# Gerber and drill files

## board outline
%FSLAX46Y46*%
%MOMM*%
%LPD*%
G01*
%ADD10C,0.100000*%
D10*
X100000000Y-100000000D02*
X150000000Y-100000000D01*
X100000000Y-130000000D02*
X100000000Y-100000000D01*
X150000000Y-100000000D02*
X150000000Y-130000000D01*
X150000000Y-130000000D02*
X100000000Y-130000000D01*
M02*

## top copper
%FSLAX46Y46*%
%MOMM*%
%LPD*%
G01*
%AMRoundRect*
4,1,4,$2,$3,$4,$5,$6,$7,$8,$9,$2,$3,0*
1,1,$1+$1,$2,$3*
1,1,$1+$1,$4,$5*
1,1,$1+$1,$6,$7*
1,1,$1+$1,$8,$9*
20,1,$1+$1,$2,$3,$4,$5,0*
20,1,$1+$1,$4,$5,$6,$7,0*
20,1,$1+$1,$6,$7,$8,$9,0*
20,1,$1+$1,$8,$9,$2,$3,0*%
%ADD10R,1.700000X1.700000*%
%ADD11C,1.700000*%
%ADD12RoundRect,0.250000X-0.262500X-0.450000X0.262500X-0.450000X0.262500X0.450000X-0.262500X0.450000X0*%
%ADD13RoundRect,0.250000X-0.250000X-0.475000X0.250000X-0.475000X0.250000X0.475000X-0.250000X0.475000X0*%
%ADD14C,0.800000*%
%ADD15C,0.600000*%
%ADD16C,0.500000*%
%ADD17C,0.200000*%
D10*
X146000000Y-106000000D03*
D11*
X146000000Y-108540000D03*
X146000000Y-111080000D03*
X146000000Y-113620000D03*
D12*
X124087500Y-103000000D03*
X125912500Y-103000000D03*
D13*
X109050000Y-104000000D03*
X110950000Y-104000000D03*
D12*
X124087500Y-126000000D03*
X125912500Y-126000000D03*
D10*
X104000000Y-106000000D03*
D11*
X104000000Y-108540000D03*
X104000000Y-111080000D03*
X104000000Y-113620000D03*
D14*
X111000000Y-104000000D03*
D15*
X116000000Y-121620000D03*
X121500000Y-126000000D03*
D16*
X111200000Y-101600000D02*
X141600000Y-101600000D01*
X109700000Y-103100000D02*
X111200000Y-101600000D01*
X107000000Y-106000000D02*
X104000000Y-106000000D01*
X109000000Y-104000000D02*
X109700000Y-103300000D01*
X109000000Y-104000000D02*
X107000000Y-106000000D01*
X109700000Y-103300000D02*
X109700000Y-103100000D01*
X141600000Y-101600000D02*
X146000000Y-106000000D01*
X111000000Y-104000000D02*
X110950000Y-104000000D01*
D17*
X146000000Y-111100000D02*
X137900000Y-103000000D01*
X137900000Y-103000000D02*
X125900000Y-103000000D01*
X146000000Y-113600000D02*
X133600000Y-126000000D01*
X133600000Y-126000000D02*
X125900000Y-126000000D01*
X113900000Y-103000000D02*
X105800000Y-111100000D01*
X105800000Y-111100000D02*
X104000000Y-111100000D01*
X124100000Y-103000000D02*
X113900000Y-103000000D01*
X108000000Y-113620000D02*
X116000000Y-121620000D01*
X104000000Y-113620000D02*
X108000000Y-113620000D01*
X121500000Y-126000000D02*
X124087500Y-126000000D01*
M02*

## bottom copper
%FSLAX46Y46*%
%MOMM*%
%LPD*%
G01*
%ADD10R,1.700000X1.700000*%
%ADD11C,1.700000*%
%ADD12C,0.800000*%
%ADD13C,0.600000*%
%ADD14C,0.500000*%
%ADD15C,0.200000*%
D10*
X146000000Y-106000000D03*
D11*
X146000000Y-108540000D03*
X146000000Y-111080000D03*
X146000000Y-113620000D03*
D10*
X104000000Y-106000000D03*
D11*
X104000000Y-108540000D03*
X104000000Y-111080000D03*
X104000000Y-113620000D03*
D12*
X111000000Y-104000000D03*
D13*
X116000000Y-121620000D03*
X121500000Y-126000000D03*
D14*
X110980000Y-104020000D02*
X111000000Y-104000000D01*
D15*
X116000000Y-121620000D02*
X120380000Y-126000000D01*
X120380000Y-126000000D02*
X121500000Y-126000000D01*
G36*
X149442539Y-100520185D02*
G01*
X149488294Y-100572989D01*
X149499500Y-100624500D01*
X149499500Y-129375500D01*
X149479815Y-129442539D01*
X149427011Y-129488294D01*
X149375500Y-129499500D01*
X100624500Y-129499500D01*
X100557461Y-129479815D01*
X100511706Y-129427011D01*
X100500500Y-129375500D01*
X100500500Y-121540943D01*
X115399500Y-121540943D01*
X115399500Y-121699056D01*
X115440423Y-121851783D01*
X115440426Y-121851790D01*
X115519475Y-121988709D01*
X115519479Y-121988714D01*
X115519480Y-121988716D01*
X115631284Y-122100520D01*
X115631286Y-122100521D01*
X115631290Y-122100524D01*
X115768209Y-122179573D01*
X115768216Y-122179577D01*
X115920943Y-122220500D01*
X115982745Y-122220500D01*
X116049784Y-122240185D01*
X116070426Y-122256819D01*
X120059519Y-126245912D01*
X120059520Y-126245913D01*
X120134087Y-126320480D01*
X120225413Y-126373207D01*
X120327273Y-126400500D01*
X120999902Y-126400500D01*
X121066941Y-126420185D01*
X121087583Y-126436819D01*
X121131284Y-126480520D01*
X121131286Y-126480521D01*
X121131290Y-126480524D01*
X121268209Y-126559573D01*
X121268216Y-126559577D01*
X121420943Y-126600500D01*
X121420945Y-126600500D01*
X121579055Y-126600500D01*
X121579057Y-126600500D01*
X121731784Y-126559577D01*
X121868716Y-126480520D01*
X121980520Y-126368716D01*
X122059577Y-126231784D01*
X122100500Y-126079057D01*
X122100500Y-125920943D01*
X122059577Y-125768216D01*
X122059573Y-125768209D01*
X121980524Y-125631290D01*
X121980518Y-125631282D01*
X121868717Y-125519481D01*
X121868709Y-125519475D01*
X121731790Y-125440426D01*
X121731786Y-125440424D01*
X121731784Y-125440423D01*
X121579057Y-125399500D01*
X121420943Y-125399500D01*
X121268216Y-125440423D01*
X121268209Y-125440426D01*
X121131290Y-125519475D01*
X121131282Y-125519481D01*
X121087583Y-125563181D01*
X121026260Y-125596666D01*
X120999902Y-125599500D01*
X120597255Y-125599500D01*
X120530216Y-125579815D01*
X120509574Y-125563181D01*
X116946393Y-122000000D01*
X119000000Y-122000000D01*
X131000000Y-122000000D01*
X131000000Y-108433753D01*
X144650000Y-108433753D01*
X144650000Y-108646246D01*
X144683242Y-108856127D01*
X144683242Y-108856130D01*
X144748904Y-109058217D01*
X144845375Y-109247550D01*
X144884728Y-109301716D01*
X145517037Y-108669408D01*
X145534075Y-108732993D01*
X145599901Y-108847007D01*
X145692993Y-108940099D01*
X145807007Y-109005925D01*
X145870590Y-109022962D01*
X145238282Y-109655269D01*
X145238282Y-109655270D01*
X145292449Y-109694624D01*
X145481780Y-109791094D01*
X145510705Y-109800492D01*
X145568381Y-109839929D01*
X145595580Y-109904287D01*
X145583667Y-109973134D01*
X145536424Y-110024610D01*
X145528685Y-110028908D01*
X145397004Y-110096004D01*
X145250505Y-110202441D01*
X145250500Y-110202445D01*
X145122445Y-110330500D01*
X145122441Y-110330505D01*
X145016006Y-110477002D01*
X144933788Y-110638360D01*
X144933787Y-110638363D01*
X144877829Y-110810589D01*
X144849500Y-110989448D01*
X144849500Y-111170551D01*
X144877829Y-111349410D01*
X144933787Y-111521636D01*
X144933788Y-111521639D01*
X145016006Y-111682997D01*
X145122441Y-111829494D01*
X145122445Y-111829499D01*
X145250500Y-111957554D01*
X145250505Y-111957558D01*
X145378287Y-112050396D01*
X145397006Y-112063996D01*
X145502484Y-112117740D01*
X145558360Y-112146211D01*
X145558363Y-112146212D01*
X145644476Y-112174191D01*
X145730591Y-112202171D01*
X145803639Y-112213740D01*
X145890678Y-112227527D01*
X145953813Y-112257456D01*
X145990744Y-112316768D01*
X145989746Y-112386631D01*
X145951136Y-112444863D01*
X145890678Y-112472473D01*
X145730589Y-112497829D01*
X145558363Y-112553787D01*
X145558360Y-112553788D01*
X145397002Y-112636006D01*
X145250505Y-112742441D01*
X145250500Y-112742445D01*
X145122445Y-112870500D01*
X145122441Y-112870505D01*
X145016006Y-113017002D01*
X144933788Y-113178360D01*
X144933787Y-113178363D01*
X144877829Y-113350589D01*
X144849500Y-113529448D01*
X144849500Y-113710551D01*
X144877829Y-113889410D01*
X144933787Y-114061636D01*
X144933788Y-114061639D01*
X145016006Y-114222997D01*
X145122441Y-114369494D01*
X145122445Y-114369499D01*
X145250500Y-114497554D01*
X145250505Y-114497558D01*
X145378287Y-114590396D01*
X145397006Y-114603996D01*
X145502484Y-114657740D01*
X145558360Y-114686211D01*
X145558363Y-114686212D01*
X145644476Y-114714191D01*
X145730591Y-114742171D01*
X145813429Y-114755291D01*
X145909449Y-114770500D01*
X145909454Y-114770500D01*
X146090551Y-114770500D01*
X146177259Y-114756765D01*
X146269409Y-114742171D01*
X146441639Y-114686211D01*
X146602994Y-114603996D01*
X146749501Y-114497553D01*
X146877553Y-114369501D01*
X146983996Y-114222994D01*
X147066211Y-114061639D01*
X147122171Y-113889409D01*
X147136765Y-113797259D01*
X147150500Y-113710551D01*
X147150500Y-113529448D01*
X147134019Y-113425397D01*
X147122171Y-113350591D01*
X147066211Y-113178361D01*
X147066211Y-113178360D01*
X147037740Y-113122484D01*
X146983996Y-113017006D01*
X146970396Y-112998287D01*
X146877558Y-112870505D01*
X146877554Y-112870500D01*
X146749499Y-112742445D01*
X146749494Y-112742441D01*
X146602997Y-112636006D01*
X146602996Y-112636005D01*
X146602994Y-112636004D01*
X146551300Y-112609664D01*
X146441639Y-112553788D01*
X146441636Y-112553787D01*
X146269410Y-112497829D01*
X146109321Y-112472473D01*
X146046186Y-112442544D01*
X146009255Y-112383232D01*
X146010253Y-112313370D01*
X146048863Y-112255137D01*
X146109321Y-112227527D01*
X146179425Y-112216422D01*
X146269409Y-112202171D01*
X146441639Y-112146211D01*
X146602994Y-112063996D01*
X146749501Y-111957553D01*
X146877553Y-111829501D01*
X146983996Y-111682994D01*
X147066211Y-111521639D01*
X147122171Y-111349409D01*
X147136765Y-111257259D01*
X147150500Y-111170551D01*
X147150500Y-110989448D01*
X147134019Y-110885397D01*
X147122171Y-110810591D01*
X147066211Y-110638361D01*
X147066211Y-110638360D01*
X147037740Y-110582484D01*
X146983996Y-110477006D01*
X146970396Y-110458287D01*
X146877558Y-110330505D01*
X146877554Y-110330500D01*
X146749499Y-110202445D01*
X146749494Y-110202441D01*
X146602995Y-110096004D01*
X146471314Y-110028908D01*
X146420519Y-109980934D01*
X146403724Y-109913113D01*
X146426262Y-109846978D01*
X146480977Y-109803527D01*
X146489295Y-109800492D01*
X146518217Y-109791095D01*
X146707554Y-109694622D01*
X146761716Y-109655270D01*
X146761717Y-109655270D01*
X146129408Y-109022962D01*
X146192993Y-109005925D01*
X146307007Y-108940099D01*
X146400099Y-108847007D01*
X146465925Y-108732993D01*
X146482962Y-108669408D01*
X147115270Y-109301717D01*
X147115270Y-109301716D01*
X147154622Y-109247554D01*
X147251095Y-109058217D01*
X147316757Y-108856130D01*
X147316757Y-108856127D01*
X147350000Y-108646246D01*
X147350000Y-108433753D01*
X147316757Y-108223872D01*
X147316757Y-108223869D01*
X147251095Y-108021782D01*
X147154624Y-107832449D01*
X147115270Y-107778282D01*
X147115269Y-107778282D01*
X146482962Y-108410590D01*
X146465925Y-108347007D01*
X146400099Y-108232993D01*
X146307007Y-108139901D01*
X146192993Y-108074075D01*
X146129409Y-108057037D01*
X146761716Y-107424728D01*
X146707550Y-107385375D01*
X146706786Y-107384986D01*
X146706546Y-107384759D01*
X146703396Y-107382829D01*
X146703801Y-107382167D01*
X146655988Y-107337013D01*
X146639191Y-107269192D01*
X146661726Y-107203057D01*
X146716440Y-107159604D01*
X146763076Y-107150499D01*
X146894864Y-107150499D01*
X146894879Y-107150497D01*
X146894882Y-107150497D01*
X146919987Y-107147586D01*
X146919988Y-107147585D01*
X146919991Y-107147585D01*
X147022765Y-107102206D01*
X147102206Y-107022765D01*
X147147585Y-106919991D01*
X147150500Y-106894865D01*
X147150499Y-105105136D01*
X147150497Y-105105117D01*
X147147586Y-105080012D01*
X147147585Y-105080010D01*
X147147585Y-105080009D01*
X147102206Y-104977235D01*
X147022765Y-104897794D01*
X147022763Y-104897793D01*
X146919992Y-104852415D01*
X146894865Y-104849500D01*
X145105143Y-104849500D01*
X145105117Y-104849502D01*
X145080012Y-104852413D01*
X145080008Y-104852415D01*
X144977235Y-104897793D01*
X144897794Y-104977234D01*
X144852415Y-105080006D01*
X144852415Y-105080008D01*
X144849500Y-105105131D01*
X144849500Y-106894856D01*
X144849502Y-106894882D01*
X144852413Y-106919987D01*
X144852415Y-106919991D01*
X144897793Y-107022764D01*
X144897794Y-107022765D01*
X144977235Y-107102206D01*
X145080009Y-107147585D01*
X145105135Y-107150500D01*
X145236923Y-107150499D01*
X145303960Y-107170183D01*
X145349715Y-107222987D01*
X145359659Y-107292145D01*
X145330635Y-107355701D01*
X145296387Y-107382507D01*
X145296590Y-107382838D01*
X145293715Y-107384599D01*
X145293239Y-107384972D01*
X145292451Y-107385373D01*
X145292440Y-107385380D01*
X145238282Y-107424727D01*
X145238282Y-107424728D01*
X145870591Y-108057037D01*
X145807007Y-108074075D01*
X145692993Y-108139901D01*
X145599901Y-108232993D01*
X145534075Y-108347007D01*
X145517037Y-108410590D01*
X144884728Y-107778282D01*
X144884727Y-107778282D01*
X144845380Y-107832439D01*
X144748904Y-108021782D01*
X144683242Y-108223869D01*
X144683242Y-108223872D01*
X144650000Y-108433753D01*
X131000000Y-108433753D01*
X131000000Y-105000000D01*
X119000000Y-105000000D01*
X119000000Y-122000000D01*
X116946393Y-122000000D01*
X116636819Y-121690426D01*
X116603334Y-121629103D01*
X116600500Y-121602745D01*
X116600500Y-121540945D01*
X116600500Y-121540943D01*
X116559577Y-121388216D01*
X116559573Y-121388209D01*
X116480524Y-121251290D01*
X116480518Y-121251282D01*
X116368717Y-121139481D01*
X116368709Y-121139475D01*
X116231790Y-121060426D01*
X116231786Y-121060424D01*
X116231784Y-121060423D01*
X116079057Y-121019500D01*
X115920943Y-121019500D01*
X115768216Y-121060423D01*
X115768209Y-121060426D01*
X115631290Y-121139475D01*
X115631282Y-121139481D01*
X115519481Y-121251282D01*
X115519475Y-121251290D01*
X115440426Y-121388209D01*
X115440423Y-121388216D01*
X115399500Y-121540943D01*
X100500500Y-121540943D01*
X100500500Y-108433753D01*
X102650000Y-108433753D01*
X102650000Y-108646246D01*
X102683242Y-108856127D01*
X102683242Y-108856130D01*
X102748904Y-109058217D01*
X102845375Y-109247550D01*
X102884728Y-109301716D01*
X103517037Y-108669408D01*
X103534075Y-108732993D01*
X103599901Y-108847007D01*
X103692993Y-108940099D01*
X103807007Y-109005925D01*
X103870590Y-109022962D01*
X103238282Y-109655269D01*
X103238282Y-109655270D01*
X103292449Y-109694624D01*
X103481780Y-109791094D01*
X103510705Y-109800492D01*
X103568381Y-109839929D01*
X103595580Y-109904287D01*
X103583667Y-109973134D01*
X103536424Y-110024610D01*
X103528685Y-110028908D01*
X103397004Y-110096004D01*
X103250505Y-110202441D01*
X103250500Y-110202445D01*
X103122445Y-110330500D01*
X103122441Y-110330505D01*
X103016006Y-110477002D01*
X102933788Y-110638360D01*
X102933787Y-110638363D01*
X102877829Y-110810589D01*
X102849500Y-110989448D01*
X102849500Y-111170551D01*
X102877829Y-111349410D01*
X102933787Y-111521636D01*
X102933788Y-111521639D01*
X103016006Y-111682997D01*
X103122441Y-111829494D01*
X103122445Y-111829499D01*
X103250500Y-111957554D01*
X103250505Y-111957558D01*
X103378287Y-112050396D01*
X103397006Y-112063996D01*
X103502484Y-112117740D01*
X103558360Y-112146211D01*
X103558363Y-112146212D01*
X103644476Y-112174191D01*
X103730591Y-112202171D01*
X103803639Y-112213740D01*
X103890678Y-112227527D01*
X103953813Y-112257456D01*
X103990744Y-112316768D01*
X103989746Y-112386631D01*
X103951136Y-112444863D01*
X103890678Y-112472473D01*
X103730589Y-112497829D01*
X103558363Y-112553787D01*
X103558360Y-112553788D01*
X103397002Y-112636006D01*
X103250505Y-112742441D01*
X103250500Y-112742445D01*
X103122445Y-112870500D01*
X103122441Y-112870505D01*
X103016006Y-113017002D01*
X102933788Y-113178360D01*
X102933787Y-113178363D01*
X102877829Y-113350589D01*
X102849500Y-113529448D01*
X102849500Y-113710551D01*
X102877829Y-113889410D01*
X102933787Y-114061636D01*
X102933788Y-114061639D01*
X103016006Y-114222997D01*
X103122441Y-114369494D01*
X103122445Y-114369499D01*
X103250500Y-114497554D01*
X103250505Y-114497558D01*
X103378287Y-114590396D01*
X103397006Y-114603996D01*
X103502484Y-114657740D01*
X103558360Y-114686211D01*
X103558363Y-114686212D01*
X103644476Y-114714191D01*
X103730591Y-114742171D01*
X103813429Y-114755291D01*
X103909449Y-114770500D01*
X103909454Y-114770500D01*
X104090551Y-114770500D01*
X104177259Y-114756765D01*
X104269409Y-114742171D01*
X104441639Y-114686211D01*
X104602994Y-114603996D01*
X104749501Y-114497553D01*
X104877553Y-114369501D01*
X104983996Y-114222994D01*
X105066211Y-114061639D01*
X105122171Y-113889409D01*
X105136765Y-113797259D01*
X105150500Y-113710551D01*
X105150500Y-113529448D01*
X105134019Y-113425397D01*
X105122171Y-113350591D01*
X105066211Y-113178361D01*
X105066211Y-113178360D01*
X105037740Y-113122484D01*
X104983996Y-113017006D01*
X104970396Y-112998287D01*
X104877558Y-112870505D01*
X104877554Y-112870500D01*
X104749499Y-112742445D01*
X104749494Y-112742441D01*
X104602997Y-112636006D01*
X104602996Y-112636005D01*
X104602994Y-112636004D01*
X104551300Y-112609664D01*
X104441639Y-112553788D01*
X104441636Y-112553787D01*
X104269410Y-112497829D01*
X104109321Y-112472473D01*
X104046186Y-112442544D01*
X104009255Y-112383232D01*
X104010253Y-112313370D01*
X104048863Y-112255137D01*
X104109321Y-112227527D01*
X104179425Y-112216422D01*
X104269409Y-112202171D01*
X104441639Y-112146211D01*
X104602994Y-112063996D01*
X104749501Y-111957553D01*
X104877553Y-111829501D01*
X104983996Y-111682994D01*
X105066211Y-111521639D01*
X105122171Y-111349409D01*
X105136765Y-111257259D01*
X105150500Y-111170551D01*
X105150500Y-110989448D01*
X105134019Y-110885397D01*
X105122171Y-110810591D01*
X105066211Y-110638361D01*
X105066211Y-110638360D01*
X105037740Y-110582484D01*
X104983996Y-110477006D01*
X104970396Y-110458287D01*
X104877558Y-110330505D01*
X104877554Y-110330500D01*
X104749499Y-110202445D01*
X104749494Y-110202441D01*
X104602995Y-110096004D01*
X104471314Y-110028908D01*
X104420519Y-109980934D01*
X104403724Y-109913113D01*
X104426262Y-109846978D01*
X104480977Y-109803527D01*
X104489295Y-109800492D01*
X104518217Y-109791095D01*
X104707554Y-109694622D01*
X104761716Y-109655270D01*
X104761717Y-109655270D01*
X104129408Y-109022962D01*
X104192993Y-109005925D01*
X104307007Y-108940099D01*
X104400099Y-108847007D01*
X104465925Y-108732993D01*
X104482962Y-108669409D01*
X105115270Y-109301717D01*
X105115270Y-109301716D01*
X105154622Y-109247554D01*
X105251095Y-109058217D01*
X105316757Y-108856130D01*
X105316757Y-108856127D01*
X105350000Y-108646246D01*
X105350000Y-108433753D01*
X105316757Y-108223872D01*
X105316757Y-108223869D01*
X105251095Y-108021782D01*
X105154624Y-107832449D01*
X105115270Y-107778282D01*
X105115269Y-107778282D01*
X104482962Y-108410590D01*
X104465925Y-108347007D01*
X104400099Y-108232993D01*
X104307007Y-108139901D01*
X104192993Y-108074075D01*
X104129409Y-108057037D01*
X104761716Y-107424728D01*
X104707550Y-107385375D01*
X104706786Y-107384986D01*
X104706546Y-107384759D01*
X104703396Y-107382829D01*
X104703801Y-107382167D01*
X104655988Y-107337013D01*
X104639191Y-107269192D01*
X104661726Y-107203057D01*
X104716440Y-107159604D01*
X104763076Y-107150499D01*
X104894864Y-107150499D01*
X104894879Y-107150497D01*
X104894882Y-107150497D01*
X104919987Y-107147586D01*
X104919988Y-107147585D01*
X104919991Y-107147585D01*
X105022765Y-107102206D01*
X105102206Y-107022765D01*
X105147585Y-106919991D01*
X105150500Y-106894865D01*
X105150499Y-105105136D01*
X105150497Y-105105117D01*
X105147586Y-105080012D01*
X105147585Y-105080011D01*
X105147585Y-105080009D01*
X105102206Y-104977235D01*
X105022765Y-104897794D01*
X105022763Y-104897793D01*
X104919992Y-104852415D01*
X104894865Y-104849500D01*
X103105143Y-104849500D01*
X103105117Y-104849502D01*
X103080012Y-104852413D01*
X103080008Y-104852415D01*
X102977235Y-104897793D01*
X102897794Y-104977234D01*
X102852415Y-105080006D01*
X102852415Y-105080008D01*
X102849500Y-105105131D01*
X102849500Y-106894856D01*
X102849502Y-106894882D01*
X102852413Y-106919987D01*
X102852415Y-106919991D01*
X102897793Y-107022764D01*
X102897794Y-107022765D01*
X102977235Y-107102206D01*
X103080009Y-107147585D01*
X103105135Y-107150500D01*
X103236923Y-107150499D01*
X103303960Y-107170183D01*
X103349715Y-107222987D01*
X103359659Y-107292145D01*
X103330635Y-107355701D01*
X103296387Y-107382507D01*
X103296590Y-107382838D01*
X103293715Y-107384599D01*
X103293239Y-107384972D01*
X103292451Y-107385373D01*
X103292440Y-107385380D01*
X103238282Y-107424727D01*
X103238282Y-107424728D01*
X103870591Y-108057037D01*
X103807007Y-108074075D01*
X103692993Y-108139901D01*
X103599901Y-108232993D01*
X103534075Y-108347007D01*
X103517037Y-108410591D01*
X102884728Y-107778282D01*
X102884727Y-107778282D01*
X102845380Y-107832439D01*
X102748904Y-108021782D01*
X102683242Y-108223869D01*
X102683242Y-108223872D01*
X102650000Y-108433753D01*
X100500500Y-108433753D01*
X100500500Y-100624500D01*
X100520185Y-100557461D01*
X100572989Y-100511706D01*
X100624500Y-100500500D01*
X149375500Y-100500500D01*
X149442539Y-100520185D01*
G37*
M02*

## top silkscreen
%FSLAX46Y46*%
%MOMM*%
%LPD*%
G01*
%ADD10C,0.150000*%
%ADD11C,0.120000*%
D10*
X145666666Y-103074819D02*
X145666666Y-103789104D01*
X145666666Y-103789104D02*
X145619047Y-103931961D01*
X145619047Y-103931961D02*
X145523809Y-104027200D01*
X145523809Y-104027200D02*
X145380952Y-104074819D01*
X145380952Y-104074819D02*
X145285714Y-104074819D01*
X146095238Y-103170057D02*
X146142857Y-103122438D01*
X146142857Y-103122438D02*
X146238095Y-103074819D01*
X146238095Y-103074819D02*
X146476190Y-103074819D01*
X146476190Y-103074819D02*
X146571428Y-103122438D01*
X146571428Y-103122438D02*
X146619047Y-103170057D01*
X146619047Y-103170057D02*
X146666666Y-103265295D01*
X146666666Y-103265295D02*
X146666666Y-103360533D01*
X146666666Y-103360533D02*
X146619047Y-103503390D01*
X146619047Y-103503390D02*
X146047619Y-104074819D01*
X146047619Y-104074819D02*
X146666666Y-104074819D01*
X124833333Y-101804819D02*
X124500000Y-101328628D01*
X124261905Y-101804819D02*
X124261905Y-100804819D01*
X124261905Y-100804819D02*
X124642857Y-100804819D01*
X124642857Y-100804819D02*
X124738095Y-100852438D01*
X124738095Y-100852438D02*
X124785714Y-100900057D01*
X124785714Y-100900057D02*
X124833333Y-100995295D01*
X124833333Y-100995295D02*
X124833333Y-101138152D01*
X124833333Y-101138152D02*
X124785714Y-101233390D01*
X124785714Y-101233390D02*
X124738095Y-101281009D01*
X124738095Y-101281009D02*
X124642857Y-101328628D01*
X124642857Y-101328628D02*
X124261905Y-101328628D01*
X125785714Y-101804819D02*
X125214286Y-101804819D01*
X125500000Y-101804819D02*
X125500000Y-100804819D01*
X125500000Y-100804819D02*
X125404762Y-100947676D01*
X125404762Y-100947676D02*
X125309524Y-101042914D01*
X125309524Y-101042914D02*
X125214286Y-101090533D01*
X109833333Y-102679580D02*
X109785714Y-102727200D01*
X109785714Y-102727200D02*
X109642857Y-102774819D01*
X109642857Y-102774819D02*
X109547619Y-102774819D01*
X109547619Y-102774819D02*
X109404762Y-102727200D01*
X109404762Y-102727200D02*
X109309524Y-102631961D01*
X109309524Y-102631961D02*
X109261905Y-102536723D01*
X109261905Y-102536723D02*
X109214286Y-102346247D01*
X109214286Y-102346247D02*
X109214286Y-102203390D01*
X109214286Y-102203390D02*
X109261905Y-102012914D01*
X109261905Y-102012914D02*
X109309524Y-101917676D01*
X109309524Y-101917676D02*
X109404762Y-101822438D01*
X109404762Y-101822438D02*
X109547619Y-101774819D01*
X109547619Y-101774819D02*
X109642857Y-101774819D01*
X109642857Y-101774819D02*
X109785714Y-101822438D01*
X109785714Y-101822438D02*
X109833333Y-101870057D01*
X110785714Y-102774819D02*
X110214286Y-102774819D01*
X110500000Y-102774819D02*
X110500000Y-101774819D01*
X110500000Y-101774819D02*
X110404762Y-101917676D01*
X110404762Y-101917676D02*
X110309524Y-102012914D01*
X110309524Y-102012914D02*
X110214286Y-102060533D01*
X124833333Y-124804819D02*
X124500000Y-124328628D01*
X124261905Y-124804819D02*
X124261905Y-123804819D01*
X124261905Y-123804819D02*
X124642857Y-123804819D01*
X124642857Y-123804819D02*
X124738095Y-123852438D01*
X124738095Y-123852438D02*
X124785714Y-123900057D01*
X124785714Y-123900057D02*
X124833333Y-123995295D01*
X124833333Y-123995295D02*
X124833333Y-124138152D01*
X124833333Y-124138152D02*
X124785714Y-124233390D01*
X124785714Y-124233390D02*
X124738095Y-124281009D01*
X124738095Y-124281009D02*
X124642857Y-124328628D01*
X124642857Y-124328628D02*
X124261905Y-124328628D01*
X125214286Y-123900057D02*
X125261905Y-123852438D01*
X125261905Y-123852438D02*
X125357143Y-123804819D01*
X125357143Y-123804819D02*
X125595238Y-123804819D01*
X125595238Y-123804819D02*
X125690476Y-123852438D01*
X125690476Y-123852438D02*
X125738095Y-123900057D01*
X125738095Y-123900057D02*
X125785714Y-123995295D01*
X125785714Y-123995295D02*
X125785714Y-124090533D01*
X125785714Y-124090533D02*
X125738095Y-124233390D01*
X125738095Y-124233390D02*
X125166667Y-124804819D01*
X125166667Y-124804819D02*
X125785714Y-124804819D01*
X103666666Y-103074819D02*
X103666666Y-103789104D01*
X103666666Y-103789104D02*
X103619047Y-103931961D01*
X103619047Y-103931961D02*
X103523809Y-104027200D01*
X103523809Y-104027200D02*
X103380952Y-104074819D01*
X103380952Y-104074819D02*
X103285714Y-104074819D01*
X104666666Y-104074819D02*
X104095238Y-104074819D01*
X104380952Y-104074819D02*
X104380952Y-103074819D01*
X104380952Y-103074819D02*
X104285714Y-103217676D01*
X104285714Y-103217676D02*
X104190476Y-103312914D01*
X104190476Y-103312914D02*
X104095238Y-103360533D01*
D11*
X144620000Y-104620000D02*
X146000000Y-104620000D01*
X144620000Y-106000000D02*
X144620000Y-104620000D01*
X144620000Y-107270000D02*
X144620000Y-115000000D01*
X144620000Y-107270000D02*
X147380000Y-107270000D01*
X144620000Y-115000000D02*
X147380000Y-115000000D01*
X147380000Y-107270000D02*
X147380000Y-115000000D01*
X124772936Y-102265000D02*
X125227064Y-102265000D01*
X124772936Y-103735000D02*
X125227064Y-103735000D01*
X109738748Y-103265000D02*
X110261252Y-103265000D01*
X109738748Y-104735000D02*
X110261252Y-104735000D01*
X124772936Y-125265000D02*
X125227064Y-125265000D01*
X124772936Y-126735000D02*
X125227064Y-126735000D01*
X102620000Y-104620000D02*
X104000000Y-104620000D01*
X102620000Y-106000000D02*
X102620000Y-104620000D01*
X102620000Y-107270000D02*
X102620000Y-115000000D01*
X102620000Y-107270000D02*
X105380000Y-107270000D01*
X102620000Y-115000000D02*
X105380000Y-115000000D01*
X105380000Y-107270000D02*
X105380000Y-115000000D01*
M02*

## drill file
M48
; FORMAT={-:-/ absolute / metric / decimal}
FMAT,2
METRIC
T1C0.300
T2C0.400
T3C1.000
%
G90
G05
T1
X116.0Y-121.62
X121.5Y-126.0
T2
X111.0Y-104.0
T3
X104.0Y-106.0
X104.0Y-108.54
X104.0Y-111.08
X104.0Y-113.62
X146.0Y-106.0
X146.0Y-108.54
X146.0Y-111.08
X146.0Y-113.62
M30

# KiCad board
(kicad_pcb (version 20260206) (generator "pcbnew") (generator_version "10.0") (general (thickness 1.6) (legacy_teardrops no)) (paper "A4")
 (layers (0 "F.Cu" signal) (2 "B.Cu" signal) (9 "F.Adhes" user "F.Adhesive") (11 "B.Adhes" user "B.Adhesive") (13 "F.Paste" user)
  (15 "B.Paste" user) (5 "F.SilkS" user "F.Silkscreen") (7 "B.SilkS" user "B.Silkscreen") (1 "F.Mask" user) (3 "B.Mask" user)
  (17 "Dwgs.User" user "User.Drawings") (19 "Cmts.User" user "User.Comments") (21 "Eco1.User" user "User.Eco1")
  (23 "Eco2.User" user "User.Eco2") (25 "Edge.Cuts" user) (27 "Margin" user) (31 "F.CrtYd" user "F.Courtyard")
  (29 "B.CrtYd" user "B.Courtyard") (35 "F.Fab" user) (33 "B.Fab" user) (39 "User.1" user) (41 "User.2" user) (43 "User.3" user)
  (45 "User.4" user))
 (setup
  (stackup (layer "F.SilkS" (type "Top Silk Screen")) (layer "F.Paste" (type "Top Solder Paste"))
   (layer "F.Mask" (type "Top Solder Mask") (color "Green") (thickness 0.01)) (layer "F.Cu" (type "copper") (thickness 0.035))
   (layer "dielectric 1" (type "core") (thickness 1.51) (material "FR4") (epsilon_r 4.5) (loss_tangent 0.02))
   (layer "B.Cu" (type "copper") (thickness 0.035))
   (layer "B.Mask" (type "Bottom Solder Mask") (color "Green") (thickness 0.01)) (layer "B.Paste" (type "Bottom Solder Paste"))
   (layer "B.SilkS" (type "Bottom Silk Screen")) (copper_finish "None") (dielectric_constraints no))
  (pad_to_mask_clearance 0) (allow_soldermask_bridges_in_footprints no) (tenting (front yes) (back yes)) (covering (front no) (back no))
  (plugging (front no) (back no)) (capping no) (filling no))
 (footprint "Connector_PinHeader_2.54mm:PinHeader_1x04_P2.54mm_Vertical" (layer "F.Cu") (at 146 106)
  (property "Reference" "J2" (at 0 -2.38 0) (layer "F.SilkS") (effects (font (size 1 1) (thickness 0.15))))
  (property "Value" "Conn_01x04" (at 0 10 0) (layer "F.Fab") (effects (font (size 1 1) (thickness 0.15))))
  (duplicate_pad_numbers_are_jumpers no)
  (fp_line (start -1.38 -1.38) (end 0 -1.38) (stroke (width 0.12) (type solid)) (layer "F.SilkS"))
  (fp_line (start -1.38 0) (end -1.38 -1.38) (stroke (width 0.12) (type solid)) (layer "F.SilkS"))
  (fp_line (start -1.38 1.27) (end -1.38 9) (stroke (width 0.12) (type solid)) (layer "F.SilkS"))
  (fp_line (start -1.38 1.27) (end 1.38 1.27) (stroke (width 0.12) (type solid)) (layer "F.SilkS"))
  (fp_line (start -1.38 9) (end 1.38 9) (stroke (width 0.12) (type solid)) (layer "F.SilkS"))
  (fp_line (start 1.38 1.27) (end 1.38 9) (stroke (width 0.12) (type solid)) (layer "F.SilkS"))
  (pad "1" thru_hole rect (at 0 0) (size 1.7 1.7) (drill 1) (layers "*.Cu" "*.Mask") (remove_unused_layers no) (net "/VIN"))
  (pad "2" thru_hole circle (at 0 2.54) (size 1.7 1.7) (drill 1) (layers "*.Cu" "*.Mask") (remove_unused_layers no) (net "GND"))
  (pad "3" thru_hole circle (at 0 5.08) (size 1.7 1.7) (drill 1) (layers "*.Cu" "*.Mask") (remove_unused_layers no) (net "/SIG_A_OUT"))
  (pad "4" thru_hole circle (at 0 7.62) (size 1.7 1.7) (drill 1) (layers "*.Cu" "*.Mask") (remove_unused_layers no) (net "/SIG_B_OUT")))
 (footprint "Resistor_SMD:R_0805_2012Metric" (layer "F.Cu") (at 125 103)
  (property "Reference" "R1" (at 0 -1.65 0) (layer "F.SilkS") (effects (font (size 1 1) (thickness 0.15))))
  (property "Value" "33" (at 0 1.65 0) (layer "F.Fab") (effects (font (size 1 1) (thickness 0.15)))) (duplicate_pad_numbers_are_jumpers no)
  (fp_line (start -0.227064 -0.735) (end 0.227064 -0.735) (stroke (width 0.12) (type solid)) (layer "F.SilkS"))
  (fp_line (start -0.227064 0.735) (end 0.227064 0.735) (stroke (width 0.12) (type solid)) (layer "F.SilkS"))
  (pad "1" smd roundrect (at -0.9125 0) (size 1.025 1.4) (layers "F.Cu" "F.Mask" "F.Paste") (roundrect_rratio 0.243902) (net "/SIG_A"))
  (pad "2" smd roundrect (at 0.9125 0) (size 1.025 1.4) (layers "F.Cu" "F.Mask" "F.Paste") (roundrect_rratio 0.243902) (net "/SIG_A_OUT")))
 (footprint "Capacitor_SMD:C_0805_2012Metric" (layer "F.Cu") (at 110 104)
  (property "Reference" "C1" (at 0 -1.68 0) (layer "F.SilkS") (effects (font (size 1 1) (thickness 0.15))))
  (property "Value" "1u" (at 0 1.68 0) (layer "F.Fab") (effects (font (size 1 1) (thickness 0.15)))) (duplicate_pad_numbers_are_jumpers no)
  (fp_line (start -0.261252 -0.735) (end 0.261252 -0.735) (stroke (width 0.12) (type solid)) (layer "F.SilkS"))
  (fp_line (start -0.261252 0.735) (end 0.261252 0.735) (stroke (width 0.12) (type solid)) (layer "F.SilkS"))
  (pad "1" smd roundrect (at -0.95 0) (size 1 1.45) (layers "F.Cu" "F.Mask" "F.Paste") (roundrect_rratio 0.25) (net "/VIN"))
  (pad "2" smd roundrect (at 0.95 0) (size 1 1.45) (layers "F.Cu" "F.Mask" "F.Paste") (roundrect_rratio 0.25) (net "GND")))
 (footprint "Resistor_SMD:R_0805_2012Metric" (layer "F.Cu") (at 125 126)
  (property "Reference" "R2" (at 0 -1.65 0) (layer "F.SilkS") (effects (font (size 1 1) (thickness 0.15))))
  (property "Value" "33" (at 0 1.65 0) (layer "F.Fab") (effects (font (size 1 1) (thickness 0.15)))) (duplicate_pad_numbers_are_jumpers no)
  (fp_line (start -0.227064 -0.735) (end 0.227064 -0.735) (stroke (width 0.12) (type solid)) (layer "F.SilkS"))
  (fp_line (start -0.227064 0.735) (end 0.227064 0.735) (stroke (width 0.12) (type solid)) (layer "F.SilkS"))
  (pad "1" smd roundrect (at -0.9125 0) (size 1.025 1.4) (layers "F.Cu" "F.Mask" "F.Paste") (roundrect_rratio 0.243902) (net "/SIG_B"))
  (pad "2" smd roundrect (at 0.9125 0) (size 1.025 1.4) (layers "F.Cu" "F.Mask" "F.Paste") (roundrect_rratio 0.243902) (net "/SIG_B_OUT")))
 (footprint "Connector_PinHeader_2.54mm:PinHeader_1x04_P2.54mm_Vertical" (layer "F.Cu") (at 104 106)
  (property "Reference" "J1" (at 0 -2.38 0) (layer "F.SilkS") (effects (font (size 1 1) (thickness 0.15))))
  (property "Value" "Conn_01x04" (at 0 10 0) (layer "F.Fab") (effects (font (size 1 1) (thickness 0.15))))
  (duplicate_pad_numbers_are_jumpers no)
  (fp_line (start -1.38 -1.38) (end 0 -1.38) (stroke (width 0.12) (type solid)) (layer "F.SilkS"))
  (fp_line (start -1.38 0) (end -1.38 -1.38) (stroke (width 0.12) (type solid)) (layer "F.SilkS"))
  (fp_line (start -1.38 1.27) (end -1.38 9) (stroke (width 0.12) (type solid)) (layer "F.SilkS"))
  (fp_line (start -1.38 1.27) (end 1.38 1.27) (stroke (width 0.12) (type solid)) (layer "F.SilkS"))
  (fp_line (start -1.38 9) (end 1.38 9) (stroke (width 0.12) (type solid)) (layer "F.SilkS"))
  (fp_line (start 1.38 1.27) (end 1.38 9) (stroke (width 0.12) (type solid)) (layer "F.SilkS"))
  (pad "1" thru_hole rect (at 0 0) (size 1.7 1.7) (drill 1) (layers "*.Cu" "*.Mask") (remove_unused_layers no) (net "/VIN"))
  (pad "2" thru_hole circle (at 0 2.54) (size 1.7 1.7) (drill 1) (layers "*.Cu" "*.Mask") (remove_unused_layers no) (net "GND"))
  (pad "3" thru_hole circle (at 0 5.08) (size 1.7 1.7) (drill 1) (layers "*.Cu" "*.Mask") (remove_unused_layers no) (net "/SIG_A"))
  (pad "4" thru_hole circle (at 0 7.62) (size 1.7 1.7) (drill 1) (layers "*.Cu" "*.Mask") (remove_unused_layers no) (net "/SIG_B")))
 (gr_line (start 100 100) (end 150 100) (stroke (width 0.1) (type default)) (layer "Edge.Cuts"))
 (gr_line (start 100 130) (end 100 100) (stroke (width 0.1) (type default)) (layer "Edge.Cuts"))
 (gr_line (start 150 100) (end 150 130) (stroke (width 0.1) (type default)) (layer "Edge.Cuts"))
 (gr_line (start 150 130) (end 100 130) (stroke (width 0.1) (type default)) (layer "Edge.Cuts"))
 (segment (start 111.2 101.6) (end 141.6 101.6) (width 0.5) (layer "F.Cu") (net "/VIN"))
 (segment (start 109.7 103.1) (end 111.2 101.6) (width 0.5) (layer "F.Cu") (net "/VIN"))
 (segment (start 107 106) (end 104 106) (width 0.5) (layer "F.Cu") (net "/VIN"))
 (segment (start 109 104) (end 109.7 103.3) (width 0.5) (layer "F.Cu") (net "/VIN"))
 (segment (start 109 104) (end 107 106) (width 0.5) (layer "F.Cu") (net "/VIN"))
 (segment (start 109.7 103.3) (end 109.7 103.1) (width 0.5) (layer "F.Cu") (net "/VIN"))
 (segment (start 141.6 101.6) (end 146 106) (width 0.5) (layer "F.Cu") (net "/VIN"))
 (segment (start 111 104) (end 110.95 104) (width 0.5) (layer "F.Cu") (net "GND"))
 (via (at 111 104) (size 0.8) (drill 0.4) (layers "F.Cu" "B.Cu") (capping yes) (filling yes) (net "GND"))
 (segment (start 110.98 104.02) (end 111 104) (width 0.5) (layer "B.Cu") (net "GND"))
 (segment (start 146 111.1) (end 137.9 103) (width 0.2) (layer "F.Cu") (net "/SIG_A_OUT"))
 (segment (start 137.9 103) (end 125.9 103) (width 0.2) (layer "F.Cu") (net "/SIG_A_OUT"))
 (segment (start 146 113.6) (end 133.6 126) (width 0.2) (layer "F.Cu") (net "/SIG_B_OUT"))
 (segment (start 133.6 126) (end 125.9 126) (width 0.2) (layer "F.Cu") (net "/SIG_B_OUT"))
 (segment (start 113.9 103) (end 105.8 111.1) (width 0.2) (layer "F.Cu") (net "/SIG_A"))
 (segment (start 105.8 111.1) (end 104 111.1) (width 0.2) (layer "F.Cu") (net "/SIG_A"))
 (segment (start 124.1 103) (end 113.9 103) (width 0.2) (layer "F.Cu") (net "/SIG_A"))
 (segment (start 108 113.62) (end 116 121.62) (width 0.2) (locked yes) (layer "F.Cu") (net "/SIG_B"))
 (segment (start 104 113.62) (end 108 113.62) (width 0.2) (locked yes) (layer "F.Cu") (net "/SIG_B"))
 (segment (start 121.5 126) (end 124.0875 126) (width 0.2) (locked yes) (layer "F.Cu") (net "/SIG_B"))
 (via (at 116 121.62) (size 0.6) (drill 0.3) (layers "F.Cu" "B.Cu") (locked yes) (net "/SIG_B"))
 (via (at 121.5 126) (size 0.6) (drill 0.3) (layers "F.Cu" "B.Cu") (locked yes) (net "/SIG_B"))
 (segment (start 116 121.62) (end 120.38 126) (width 0.2) (locked yes) (layer "B.Cu") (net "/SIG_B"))
 (segment (start 120.38 126) (end 121.5 126) (width 0.2) (locked yes) (layer "B.Cu") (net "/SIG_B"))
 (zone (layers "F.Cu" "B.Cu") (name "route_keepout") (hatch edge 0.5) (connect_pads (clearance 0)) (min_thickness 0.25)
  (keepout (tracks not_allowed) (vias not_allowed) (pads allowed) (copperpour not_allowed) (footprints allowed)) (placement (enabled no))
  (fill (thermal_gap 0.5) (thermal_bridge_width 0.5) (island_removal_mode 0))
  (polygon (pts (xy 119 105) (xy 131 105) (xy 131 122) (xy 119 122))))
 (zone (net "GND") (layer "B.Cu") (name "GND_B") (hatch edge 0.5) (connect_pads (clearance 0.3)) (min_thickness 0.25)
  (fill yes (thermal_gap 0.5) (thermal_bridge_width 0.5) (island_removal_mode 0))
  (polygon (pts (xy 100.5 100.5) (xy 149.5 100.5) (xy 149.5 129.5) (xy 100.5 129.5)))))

